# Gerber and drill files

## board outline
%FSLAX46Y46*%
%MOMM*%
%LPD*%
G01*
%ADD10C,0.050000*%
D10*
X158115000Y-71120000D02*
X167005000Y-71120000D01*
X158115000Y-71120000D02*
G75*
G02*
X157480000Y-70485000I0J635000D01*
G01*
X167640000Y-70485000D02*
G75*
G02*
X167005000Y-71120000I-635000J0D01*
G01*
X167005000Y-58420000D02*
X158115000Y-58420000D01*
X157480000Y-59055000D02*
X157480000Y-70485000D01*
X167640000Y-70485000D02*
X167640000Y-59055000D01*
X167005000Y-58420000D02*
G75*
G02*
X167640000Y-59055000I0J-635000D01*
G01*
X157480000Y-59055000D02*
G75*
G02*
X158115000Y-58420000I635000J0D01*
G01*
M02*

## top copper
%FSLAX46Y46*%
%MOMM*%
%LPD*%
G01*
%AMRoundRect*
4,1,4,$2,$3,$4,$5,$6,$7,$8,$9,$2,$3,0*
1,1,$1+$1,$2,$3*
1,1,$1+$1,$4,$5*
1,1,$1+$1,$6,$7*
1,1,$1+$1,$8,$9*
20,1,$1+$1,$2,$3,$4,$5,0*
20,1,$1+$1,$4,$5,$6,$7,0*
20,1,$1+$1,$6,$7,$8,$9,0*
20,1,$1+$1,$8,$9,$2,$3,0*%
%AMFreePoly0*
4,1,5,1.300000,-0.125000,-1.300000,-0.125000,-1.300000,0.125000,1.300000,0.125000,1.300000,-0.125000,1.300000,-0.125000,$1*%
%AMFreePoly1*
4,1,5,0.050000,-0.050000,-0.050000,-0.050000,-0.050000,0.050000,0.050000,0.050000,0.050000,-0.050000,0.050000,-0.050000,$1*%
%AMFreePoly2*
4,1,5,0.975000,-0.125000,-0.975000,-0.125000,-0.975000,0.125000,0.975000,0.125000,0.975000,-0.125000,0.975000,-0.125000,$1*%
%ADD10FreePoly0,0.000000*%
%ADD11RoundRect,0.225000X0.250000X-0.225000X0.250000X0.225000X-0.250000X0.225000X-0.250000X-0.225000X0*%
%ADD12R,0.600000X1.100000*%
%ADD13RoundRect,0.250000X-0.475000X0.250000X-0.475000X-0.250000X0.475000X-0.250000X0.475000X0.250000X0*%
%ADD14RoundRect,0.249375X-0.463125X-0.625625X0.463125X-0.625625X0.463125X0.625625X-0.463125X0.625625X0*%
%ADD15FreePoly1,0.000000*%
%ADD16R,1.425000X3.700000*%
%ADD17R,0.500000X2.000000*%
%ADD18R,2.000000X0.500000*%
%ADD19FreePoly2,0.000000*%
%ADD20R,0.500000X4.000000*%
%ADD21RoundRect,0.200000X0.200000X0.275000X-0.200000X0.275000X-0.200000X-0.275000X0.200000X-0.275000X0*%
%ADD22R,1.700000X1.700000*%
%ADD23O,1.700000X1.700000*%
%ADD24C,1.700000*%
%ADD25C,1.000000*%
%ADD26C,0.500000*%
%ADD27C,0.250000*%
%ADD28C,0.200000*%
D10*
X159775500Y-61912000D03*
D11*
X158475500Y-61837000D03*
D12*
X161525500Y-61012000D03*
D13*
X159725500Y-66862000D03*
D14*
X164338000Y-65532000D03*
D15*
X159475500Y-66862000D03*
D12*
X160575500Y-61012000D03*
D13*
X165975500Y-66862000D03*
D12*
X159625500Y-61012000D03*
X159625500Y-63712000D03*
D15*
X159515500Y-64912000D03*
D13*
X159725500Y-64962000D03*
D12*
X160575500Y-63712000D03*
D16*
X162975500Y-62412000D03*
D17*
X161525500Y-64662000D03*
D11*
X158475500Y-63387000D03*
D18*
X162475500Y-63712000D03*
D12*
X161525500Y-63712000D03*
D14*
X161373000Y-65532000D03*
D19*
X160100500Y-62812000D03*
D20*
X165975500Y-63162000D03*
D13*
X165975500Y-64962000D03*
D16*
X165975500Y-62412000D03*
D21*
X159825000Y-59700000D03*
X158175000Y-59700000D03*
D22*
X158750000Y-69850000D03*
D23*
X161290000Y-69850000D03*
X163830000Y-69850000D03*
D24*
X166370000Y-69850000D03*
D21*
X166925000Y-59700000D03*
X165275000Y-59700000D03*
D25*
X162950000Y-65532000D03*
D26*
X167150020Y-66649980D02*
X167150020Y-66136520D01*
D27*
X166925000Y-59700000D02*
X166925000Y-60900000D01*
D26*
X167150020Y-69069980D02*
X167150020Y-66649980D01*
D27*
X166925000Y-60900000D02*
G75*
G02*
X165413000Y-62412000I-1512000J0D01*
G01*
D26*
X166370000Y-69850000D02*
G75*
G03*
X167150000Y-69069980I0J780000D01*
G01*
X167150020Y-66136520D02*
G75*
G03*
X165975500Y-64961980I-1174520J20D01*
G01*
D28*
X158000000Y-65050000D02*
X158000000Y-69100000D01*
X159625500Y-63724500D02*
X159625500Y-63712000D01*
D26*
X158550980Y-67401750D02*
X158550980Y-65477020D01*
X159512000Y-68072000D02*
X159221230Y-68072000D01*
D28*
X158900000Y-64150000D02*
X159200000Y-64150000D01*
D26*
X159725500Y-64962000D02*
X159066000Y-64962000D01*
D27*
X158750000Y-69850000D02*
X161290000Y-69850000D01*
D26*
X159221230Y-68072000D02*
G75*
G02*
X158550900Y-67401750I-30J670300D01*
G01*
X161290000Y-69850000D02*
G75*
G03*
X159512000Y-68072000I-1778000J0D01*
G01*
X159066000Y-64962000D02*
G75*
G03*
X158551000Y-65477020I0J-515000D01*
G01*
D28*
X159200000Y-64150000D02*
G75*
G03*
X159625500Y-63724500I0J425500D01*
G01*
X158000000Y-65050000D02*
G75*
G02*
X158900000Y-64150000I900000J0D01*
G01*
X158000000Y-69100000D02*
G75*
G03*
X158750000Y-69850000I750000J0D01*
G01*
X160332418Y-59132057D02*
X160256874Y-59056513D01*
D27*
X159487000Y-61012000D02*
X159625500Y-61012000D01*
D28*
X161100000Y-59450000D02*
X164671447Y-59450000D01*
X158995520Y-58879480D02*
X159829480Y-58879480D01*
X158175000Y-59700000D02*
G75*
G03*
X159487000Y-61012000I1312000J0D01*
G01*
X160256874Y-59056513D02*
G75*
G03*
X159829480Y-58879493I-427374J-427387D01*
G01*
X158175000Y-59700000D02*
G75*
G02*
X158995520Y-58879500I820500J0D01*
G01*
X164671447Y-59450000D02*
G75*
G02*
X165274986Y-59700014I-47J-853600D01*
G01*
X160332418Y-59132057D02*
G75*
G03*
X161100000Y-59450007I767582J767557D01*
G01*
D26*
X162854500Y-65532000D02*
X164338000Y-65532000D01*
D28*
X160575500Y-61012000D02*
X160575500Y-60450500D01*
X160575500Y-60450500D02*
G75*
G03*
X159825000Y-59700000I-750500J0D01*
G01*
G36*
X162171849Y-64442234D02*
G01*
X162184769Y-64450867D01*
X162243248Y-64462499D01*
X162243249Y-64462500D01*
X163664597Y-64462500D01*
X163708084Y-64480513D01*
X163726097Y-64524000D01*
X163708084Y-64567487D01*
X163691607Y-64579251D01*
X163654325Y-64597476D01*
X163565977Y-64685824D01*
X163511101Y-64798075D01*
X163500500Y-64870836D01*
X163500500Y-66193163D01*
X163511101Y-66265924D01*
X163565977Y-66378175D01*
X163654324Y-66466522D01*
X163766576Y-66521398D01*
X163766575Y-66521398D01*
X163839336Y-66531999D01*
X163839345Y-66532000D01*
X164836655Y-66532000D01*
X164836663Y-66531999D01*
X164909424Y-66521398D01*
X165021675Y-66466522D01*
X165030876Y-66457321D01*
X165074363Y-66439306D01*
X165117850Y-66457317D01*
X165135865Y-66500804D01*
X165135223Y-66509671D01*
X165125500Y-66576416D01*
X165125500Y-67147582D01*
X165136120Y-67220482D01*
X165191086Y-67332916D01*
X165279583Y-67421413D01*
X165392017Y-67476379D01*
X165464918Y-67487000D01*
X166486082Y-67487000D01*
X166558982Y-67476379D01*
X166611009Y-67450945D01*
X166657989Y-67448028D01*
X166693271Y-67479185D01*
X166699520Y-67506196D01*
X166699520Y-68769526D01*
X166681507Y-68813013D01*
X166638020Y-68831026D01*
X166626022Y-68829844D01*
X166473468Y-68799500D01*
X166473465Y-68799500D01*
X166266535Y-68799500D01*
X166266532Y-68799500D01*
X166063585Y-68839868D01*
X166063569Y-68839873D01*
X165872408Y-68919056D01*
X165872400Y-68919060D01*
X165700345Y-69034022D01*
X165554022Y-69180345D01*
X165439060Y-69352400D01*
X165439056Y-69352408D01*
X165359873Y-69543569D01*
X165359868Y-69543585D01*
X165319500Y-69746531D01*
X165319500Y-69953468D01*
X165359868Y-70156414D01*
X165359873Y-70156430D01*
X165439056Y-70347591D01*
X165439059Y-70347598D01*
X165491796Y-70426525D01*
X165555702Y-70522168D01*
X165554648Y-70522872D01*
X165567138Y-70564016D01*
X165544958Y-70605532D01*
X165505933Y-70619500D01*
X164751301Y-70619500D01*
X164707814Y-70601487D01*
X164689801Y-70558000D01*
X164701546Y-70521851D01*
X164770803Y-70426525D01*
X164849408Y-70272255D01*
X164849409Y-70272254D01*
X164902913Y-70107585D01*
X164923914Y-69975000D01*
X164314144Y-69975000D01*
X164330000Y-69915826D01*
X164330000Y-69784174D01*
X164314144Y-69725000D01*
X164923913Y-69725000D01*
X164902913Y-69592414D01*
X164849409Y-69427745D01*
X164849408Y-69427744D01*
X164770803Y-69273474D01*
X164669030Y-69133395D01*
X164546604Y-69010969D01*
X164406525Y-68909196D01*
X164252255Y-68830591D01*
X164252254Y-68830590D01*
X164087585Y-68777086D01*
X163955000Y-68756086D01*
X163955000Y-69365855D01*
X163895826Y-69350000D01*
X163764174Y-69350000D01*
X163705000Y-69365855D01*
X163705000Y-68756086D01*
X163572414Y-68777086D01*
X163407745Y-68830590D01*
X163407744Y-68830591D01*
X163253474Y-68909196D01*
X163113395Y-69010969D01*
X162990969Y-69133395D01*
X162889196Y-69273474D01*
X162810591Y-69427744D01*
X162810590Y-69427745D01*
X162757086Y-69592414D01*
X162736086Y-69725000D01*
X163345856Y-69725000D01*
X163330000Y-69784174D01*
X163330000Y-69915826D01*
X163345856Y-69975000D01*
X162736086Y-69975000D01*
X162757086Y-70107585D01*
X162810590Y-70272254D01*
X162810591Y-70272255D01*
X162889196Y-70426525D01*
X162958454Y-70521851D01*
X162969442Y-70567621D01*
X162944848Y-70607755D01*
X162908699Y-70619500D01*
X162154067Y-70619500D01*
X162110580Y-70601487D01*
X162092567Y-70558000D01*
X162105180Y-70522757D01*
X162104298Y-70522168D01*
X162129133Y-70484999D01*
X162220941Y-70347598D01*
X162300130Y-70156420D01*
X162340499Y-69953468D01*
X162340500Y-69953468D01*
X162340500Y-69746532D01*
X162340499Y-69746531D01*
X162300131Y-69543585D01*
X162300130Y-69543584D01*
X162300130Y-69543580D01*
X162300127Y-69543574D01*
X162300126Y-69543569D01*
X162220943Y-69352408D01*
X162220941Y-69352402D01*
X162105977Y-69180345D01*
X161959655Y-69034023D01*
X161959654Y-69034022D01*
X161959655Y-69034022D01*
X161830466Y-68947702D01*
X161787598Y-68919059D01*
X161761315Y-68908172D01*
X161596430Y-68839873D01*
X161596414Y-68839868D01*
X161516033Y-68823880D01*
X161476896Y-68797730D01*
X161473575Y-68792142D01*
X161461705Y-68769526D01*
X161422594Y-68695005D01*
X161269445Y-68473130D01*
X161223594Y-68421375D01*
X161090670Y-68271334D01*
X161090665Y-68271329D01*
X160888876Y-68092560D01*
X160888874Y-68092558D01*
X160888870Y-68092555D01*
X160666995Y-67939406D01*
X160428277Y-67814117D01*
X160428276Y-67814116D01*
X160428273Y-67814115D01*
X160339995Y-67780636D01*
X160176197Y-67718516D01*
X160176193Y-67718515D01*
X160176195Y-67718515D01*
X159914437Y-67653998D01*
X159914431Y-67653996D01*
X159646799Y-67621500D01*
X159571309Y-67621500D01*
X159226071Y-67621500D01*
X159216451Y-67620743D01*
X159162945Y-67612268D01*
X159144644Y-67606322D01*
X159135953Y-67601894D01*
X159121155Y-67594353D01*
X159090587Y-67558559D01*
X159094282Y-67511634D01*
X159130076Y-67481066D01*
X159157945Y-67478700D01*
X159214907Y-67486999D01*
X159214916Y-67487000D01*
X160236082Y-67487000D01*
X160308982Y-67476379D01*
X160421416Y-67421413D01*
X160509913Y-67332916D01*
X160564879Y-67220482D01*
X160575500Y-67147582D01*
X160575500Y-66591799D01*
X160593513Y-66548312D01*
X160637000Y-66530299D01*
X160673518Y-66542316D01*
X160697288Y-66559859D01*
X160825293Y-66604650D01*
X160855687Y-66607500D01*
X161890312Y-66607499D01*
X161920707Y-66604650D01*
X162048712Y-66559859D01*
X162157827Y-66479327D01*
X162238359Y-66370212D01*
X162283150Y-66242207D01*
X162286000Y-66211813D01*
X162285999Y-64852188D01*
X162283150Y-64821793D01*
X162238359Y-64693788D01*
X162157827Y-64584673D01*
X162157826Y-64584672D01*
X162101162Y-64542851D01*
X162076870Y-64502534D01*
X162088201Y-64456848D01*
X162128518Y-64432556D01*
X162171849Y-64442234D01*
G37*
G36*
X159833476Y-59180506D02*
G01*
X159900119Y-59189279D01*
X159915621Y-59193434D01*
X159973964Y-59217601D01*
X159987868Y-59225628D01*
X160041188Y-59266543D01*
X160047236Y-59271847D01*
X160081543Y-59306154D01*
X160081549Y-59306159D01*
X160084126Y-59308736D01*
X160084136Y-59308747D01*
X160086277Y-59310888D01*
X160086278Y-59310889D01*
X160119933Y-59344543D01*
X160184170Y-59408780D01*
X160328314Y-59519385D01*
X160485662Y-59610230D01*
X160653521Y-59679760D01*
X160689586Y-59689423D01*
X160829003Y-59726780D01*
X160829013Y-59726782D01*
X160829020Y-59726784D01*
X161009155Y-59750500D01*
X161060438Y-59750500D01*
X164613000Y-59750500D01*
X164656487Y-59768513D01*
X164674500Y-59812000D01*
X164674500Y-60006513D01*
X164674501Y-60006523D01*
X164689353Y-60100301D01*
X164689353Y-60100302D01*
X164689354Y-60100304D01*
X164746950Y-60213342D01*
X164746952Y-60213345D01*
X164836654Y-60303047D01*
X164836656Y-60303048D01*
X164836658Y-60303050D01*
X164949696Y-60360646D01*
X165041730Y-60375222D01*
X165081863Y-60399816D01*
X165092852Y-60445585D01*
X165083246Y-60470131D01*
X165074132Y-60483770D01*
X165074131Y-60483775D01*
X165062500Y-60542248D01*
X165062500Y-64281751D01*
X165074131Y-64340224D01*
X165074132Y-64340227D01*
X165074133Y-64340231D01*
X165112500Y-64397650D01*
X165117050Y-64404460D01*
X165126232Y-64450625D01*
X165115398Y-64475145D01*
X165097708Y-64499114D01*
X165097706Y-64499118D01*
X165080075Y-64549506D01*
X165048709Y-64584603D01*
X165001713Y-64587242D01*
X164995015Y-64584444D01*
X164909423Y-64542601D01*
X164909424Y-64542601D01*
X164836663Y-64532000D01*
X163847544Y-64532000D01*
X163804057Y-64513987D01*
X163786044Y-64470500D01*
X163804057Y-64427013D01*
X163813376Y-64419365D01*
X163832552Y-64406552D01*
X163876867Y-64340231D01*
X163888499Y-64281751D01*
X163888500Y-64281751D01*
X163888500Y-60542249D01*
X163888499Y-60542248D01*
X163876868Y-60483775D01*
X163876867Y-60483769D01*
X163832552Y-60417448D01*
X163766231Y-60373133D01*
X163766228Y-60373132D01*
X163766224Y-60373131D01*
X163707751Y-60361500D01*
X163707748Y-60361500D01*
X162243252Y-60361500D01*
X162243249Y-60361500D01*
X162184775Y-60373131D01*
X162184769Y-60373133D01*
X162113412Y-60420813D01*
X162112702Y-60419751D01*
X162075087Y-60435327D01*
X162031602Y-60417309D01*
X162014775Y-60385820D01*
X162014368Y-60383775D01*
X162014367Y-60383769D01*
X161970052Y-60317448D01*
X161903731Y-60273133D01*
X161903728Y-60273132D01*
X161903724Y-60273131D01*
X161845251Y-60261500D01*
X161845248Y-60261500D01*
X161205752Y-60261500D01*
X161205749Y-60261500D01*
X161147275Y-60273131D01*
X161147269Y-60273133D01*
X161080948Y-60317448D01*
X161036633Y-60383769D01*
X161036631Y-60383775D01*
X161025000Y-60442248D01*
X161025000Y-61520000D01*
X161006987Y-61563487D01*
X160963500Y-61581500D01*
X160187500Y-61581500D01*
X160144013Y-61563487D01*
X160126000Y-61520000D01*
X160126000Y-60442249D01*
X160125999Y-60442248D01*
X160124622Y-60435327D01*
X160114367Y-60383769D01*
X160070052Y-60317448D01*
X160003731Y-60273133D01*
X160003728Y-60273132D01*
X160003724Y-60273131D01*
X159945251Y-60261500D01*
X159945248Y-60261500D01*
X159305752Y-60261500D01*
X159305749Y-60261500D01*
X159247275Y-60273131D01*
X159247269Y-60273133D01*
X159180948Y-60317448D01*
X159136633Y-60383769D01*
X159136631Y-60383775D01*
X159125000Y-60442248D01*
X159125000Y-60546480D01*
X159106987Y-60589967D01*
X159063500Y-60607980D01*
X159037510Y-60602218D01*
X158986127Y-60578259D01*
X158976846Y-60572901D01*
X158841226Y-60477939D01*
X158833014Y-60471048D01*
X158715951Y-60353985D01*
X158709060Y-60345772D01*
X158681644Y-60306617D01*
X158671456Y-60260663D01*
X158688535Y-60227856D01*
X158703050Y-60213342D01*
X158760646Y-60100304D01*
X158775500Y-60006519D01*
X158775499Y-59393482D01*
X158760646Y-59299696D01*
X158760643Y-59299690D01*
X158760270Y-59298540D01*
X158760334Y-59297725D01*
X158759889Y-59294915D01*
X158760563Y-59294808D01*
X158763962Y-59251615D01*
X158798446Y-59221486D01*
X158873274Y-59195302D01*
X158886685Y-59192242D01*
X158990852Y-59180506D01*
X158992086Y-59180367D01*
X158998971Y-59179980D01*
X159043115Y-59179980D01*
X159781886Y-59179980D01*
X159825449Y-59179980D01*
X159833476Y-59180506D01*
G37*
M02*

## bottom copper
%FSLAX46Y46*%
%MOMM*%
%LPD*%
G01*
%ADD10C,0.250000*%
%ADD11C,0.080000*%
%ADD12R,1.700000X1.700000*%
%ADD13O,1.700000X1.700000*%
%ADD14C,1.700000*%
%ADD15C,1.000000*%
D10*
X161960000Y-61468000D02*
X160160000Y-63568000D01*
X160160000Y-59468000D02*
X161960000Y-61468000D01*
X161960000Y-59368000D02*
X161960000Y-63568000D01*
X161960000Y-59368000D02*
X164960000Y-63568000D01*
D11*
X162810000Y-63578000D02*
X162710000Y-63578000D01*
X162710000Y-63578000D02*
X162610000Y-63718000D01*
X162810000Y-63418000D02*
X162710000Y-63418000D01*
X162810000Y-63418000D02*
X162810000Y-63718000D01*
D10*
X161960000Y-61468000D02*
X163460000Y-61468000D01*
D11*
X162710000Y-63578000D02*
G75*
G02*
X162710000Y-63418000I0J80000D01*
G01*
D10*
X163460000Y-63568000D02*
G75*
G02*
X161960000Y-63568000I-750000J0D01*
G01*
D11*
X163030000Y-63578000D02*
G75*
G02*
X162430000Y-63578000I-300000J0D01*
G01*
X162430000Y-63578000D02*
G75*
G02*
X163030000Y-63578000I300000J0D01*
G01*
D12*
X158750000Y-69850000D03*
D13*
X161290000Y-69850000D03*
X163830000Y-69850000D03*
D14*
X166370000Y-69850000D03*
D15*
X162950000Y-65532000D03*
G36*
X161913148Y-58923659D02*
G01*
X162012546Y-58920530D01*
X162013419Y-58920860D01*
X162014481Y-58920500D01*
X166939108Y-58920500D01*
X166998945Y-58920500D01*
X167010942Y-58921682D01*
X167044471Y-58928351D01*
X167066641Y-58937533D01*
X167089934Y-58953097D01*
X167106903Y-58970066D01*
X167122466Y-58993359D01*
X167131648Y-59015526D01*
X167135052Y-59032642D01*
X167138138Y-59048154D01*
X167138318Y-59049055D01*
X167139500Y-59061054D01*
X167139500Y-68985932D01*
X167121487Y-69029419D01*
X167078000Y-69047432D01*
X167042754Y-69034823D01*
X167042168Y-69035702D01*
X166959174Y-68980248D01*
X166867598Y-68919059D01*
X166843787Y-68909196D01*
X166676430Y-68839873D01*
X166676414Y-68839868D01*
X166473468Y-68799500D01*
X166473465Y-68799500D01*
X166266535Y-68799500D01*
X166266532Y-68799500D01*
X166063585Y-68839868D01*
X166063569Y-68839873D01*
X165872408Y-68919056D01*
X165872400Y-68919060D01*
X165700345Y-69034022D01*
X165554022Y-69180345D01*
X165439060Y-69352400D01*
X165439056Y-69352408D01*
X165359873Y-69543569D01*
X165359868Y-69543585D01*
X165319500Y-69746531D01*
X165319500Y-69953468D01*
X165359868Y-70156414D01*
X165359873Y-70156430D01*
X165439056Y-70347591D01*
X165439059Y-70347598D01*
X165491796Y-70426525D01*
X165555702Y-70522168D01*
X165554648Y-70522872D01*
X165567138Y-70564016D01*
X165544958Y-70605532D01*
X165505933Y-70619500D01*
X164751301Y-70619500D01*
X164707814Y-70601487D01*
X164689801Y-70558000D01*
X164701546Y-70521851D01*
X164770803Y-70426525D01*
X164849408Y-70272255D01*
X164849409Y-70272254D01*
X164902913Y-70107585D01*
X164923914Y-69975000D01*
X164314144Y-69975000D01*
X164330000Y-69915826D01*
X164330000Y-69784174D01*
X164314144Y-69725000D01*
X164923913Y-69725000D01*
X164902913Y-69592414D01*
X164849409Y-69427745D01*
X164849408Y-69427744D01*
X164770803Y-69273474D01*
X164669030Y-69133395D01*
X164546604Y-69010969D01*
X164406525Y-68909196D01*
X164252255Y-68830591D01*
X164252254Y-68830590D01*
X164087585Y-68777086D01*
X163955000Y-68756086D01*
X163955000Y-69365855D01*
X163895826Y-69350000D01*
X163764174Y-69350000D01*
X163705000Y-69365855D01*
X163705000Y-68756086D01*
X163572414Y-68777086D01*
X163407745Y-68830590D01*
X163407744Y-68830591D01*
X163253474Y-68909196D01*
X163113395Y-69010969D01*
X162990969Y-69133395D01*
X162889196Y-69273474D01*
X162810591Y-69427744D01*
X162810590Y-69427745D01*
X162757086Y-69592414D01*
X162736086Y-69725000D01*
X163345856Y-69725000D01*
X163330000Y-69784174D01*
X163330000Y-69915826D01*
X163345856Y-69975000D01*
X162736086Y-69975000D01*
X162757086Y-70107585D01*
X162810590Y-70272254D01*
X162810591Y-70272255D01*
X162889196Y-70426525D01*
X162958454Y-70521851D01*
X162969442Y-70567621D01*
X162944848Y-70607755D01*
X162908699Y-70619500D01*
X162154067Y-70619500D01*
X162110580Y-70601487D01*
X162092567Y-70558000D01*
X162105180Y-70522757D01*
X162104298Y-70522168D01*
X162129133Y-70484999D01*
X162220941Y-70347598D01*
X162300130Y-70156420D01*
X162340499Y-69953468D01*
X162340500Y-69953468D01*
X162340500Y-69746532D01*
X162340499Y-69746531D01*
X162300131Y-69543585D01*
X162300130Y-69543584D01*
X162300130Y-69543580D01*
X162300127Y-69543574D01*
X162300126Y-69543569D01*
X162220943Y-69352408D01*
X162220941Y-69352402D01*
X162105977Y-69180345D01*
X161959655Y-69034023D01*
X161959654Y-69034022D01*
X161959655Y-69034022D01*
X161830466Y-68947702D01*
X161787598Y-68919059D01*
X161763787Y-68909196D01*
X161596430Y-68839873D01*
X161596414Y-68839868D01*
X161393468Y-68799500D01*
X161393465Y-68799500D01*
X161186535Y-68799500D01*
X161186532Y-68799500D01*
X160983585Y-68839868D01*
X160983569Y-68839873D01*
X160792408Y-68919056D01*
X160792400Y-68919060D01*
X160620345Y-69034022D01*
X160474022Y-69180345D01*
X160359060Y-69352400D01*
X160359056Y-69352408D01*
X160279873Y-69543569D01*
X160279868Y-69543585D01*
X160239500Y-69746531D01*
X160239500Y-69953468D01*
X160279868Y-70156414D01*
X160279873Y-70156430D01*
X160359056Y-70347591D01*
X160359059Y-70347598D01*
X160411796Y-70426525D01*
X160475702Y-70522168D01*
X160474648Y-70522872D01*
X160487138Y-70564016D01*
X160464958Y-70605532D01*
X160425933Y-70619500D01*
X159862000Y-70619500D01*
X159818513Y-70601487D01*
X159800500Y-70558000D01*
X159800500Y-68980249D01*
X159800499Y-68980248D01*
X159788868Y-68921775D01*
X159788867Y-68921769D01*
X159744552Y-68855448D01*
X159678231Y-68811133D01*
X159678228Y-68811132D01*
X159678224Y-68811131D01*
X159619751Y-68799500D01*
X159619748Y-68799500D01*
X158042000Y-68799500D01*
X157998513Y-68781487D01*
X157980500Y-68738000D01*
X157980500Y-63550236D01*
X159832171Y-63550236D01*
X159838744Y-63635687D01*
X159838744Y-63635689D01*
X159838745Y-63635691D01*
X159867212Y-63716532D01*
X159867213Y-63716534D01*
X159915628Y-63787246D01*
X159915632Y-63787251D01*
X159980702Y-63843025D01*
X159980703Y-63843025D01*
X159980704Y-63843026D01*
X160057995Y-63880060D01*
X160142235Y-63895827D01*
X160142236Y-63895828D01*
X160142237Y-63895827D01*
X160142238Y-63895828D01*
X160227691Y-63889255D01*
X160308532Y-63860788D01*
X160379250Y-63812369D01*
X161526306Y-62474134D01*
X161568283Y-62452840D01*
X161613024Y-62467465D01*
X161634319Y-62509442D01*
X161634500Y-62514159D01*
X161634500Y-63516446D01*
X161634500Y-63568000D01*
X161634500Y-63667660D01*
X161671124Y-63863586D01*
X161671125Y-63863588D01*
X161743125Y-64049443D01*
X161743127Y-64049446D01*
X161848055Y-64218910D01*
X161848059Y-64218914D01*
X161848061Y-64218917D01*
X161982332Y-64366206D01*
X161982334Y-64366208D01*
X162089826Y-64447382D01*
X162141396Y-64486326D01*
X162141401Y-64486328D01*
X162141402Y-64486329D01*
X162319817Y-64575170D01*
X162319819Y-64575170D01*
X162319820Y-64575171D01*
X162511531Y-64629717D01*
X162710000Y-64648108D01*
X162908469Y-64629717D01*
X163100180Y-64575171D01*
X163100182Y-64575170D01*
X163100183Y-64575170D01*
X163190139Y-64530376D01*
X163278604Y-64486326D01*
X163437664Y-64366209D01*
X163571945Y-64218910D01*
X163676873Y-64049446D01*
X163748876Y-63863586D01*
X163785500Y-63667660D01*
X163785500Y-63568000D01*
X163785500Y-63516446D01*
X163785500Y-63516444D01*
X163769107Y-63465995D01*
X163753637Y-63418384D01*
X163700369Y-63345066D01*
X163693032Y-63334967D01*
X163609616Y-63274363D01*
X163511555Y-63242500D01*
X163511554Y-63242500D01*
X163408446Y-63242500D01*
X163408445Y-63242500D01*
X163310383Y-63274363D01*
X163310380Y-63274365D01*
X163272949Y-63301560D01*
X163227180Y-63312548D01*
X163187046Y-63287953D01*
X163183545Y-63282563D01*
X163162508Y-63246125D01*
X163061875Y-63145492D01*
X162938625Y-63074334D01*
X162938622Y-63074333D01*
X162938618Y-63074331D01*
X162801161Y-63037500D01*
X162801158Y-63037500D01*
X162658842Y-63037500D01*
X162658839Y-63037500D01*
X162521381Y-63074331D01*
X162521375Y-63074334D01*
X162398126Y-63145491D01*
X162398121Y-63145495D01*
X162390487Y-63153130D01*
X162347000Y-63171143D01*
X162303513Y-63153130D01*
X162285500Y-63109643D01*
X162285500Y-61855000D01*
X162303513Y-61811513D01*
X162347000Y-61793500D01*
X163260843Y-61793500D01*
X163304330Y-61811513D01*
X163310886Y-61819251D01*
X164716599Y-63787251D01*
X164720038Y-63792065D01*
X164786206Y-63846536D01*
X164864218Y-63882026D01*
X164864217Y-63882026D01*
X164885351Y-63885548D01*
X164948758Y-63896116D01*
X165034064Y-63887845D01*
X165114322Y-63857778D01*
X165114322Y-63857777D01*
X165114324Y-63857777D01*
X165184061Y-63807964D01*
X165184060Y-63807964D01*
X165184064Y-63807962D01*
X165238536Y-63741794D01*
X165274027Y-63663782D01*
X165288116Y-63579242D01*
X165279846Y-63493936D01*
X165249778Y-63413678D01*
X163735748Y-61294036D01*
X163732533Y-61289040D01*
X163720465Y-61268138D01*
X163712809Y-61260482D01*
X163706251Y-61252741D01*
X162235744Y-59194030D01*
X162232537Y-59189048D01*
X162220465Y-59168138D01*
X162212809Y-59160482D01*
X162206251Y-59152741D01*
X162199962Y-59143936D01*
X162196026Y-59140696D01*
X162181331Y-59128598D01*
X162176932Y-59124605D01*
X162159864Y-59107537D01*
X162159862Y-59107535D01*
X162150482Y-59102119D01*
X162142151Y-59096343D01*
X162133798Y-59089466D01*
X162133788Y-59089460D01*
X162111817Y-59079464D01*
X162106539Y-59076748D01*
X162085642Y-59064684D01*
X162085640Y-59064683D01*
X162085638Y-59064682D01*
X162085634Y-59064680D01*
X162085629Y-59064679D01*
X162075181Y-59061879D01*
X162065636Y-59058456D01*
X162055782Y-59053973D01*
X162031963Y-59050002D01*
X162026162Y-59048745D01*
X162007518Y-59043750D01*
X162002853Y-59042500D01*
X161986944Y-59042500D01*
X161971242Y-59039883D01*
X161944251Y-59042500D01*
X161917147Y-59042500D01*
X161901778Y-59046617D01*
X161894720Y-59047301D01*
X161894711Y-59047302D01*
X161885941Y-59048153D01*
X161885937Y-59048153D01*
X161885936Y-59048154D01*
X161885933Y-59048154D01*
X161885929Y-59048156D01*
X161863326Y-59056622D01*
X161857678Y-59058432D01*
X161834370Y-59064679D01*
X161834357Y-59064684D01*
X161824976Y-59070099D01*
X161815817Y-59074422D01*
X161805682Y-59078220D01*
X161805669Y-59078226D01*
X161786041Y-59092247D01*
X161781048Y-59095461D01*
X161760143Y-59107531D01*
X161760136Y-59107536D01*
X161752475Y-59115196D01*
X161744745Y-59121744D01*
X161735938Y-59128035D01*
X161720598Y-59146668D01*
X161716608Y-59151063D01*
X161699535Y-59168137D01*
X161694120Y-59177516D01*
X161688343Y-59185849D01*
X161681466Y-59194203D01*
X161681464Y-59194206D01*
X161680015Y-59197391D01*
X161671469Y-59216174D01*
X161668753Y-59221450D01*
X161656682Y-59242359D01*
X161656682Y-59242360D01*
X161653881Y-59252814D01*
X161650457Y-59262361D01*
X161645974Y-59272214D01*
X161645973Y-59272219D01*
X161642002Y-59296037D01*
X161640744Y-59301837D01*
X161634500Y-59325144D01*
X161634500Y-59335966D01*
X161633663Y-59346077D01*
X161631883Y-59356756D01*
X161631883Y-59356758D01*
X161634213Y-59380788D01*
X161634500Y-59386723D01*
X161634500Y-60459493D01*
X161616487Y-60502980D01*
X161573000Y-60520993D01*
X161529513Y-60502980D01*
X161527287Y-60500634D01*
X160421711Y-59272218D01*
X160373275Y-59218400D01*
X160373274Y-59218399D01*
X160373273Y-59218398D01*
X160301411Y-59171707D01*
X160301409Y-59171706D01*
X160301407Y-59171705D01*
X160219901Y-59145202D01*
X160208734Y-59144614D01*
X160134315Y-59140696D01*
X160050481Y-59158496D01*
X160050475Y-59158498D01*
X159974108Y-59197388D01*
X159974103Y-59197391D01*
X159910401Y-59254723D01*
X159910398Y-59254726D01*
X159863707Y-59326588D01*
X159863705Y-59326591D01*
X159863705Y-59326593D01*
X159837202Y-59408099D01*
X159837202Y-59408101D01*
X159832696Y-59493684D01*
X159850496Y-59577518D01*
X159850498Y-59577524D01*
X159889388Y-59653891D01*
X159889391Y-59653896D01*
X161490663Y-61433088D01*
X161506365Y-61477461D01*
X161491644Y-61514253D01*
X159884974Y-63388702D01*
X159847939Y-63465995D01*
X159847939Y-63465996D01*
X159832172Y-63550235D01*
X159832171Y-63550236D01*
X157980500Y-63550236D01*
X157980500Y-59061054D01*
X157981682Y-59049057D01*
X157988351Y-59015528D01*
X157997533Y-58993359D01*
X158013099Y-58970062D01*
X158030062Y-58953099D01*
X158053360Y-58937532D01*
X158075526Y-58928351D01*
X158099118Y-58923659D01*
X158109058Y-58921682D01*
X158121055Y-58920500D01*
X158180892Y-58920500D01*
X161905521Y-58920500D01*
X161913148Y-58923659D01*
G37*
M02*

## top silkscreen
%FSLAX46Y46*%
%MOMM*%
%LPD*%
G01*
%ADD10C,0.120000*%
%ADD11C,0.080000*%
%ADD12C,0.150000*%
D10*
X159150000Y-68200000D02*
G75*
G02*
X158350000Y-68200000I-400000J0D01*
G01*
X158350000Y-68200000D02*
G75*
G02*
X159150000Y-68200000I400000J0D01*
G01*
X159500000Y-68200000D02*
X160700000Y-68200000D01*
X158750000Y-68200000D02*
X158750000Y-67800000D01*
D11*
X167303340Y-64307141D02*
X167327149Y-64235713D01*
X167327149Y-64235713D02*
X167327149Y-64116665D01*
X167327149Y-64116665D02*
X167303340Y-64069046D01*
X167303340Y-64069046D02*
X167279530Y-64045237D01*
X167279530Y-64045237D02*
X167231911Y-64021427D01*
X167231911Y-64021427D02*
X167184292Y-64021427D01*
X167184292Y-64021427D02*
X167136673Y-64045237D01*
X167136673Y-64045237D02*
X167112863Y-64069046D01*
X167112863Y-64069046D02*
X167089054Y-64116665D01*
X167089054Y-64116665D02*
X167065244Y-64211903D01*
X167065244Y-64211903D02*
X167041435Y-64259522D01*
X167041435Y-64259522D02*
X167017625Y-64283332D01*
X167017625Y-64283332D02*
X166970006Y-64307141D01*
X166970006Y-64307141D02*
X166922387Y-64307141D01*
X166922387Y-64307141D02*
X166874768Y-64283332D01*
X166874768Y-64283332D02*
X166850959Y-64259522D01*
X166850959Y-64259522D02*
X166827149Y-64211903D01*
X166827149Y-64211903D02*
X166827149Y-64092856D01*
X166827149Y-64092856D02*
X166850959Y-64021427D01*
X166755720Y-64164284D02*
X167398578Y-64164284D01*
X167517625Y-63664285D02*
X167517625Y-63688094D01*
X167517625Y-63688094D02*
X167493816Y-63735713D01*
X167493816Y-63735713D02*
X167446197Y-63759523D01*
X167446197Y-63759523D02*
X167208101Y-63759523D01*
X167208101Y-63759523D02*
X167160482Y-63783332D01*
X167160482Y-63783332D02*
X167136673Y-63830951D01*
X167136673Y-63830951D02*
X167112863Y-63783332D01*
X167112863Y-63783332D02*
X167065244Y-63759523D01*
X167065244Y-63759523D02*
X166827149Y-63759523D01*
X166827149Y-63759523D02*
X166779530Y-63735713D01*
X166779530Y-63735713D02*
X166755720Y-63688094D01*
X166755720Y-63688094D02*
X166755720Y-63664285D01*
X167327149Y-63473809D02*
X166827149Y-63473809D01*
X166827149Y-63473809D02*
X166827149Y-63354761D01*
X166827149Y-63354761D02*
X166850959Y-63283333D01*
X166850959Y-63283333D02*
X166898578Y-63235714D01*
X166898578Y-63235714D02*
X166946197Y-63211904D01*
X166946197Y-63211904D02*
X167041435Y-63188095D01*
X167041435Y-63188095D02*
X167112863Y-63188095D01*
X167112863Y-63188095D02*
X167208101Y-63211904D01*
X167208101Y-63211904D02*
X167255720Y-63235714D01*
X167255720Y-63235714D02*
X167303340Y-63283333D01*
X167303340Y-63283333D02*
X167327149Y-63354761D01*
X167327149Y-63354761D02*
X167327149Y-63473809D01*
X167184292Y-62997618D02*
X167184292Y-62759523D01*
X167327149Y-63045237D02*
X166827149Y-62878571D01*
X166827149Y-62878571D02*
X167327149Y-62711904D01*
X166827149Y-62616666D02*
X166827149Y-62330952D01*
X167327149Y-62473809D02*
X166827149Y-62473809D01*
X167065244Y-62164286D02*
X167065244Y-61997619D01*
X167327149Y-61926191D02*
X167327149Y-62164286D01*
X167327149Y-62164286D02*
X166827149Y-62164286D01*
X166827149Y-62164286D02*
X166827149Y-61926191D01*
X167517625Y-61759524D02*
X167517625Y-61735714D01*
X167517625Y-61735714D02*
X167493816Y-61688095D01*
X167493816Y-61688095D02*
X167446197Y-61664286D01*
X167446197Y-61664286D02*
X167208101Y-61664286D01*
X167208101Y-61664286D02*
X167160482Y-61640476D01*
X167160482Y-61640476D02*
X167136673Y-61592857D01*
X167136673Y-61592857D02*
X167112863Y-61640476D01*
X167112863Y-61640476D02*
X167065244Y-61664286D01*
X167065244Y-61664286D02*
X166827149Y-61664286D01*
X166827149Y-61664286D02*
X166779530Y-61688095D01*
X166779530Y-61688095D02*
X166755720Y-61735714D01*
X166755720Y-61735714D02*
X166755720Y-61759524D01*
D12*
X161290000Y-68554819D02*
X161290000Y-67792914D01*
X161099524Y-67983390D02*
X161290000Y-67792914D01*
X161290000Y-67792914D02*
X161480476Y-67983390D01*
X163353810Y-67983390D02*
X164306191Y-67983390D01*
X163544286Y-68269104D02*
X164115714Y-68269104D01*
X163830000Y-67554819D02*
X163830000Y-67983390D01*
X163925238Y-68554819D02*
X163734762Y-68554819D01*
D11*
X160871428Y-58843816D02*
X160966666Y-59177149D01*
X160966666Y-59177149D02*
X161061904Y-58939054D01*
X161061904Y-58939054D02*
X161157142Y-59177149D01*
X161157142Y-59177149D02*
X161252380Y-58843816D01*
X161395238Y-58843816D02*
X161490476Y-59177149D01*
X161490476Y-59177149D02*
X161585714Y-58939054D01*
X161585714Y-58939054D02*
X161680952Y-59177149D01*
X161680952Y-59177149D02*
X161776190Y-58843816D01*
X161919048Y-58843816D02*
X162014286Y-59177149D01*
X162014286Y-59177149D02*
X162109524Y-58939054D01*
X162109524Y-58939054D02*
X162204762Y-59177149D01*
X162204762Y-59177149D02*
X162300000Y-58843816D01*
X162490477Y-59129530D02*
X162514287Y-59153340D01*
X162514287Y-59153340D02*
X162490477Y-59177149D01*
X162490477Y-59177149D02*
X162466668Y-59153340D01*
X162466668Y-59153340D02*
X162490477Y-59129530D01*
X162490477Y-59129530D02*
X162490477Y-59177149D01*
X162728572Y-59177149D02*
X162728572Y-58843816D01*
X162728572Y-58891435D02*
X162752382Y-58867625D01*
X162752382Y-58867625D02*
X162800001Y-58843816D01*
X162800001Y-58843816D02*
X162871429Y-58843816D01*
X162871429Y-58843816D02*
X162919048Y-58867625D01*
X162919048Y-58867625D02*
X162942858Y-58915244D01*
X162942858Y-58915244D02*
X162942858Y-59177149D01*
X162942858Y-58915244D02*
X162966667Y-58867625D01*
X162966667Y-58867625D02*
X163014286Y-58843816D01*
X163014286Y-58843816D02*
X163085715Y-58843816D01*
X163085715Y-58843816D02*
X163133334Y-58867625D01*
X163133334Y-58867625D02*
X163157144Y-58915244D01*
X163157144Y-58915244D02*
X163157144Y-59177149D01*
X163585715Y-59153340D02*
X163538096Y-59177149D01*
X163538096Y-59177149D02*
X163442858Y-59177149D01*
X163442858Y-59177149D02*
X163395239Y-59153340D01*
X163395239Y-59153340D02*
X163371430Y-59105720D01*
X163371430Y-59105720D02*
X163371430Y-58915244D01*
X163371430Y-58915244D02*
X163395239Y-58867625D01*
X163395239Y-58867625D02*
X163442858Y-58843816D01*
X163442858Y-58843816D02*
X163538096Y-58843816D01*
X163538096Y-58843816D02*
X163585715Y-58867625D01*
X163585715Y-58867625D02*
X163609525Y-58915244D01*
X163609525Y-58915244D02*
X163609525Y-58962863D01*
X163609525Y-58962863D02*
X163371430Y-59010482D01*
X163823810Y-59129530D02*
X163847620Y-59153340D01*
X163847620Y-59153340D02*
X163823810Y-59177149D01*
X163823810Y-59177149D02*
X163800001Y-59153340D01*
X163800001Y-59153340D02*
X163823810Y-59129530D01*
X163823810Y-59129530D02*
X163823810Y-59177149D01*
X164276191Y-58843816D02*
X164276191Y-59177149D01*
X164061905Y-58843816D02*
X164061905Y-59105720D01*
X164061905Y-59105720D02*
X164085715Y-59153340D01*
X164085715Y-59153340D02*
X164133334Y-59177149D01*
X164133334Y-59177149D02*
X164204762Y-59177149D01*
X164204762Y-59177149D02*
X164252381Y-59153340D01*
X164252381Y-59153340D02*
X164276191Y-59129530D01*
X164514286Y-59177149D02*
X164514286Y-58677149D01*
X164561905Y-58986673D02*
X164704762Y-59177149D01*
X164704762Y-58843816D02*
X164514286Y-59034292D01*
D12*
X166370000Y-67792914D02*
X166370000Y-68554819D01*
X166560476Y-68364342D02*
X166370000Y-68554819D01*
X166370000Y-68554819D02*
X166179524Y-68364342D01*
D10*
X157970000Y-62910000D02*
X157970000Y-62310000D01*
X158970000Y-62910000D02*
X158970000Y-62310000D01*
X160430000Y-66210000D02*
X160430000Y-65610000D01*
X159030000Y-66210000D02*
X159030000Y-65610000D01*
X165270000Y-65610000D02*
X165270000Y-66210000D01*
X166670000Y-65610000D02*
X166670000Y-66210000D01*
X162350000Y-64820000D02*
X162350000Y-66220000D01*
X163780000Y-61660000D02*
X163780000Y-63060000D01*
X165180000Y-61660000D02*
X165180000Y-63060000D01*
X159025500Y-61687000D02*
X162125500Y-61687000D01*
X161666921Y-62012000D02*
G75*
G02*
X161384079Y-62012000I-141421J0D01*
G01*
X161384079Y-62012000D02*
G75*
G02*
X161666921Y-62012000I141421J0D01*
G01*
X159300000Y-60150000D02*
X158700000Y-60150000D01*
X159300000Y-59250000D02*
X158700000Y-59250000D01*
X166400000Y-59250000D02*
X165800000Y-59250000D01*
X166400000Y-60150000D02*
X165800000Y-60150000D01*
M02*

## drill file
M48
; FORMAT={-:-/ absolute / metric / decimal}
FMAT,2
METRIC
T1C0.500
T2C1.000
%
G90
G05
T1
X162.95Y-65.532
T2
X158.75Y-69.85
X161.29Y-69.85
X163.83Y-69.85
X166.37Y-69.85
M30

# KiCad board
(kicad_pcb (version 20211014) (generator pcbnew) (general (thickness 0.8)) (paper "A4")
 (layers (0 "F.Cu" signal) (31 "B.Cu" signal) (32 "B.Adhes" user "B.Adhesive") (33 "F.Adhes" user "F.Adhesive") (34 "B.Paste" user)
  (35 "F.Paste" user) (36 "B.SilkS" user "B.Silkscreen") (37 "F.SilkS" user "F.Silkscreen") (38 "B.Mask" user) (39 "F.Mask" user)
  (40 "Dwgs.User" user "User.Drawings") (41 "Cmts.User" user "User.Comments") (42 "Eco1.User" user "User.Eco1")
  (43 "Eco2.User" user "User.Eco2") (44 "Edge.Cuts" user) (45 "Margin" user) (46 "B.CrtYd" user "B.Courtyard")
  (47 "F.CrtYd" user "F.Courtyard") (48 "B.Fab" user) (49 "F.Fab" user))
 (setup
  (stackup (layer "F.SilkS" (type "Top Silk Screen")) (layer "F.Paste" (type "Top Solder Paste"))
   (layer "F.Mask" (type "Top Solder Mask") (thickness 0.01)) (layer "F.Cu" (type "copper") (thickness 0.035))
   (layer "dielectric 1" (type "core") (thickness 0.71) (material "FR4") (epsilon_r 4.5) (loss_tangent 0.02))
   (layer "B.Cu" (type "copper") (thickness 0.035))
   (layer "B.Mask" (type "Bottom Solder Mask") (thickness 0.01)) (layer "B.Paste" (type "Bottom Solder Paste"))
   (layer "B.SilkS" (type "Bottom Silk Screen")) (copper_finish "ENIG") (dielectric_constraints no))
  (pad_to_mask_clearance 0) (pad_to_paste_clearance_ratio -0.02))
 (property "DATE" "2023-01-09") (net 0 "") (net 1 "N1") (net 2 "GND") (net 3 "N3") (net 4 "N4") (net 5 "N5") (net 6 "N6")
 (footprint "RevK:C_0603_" (layer "F.Cu") (at 158.47 62.61 90)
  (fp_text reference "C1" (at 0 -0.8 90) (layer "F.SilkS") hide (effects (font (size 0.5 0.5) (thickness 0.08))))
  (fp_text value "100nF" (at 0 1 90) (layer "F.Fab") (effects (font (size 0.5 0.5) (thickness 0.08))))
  (fp_line (start -0.3 -0.5) (end 0.3 -0.5) (layer "F.SilkS") (width 0.12))
  (fp_line (start -0.3 0.5) (end 0.3 0.5) (layer "F.SilkS") (width 0.12)))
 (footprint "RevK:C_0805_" (layer "F.Cu") (at 159.73 65.91 90)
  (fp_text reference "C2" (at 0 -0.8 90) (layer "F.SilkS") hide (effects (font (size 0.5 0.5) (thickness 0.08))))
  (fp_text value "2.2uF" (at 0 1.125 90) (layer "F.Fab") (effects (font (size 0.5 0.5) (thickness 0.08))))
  (fp_line (start -0.3 0.7) (end 0.3 0.7) (layer "F.SilkS") (width 0.12))
  (fp_line (start -0.3 -0.7) (end 0.3 -0.7) (layer "F.SilkS") (width 0.12)))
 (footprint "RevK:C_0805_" (layer "F.Cu") (at 165.97 65.91 -90)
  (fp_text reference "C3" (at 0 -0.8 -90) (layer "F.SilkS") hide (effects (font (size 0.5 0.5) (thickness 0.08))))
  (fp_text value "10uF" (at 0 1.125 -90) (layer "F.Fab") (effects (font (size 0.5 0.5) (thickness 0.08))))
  (fp_line (start -0.3 0.7) (end 0.3 0.7) (layer "F.SilkS") (width 0.12))
  (fp_line (start -0.3 -0.7) (end 0.3 -0.7) (layer "F.SilkS") (width 0.12)))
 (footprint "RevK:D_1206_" (layer "F.Cu") (at 162.85 65.52)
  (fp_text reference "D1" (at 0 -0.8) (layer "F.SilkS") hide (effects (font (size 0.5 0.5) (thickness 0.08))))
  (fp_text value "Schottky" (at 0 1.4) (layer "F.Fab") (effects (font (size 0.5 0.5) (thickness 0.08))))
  (fp_line (start -0.5 -0.7) (end -0.5 0.7) (layer "F.SilkS") (width 0.12)))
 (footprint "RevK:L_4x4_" (layer "F.Cu") (at 164.48 62.36)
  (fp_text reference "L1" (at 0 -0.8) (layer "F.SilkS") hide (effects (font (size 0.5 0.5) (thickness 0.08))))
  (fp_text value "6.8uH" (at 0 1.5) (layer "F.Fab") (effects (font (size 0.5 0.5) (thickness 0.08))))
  (fp_line (start -0.7 -0.7) (end -0.7 0.7) (layer "F.SilkS") (width 0.12))
  (fp_line (start 0.7 -0.7) (end 0.7 0.7) (layer "F.SilkS") (width 0.12)))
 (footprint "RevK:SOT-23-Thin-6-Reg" (layer "F.Cu") (at 160.5755 62.362)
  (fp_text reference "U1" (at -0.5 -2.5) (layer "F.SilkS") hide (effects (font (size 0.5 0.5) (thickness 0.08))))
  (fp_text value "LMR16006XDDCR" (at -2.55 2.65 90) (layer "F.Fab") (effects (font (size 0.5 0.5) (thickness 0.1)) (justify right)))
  (fp_line (start -1.55 -0.675) (end 1.55 -0.675) (layer "F.SilkS") (width 0.12))
  (fp_circle (center 0.95 -0.35) (end 1.05 -0.25) (layer "F.SilkS") (width 0.12) (fill none))
  (pad "" smd roundrect (at 5.4 0.05) (size 1.2 1) (layers "F.Paste") (roundrect_rratio 0.25))
  (pad "" smd roundrect (at 5.4 1.2) (size 1.2 1) (layers "F.Paste") (roundrect_rratio 0.25))
  (pad "" smd roundrect (at 2.4 0.05) (size 1.2 1) (layers "F.Paste") (roundrect_rratio 0.25))
  (pad "" smd roundrect (at 2.4 1.2) (size 1.2 1) (layers "F.Paste") (roundrect_rratio 0.25))
  (pad "" smd roundrect (at 2.4 -1.1) (size 1.2 1) (layers "F.Paste") (roundrect_rratio 0.25))
  (pad "" smd roundrect (at 5.4 -1.1) (size 1.2 1) (layers "F.Paste") (roundrect_rratio 0.25))
  (pad "1" smd custom (at -0.8 -0.45) (size 2.6 0.25) (layers "F.Cu") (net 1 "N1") (clearance 0.2)
   (options (clearance outline) (anchor rect)) (primitives))
  (pad "1" smd roundrect (at -2.1 -0.525 90) (size 0.9 0.95) (layers "F.Cu" "F.Paste" "F.Mask") (roundrect_rratio 0.25) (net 1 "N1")
   (clearance 0.2))
  (pad "1" smd rect (at 0.95 -1.35 90) (size 1.1 0.6) (layers "F.Cu" "F.Paste" "F.Mask") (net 1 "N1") (clearance 0.2))
  (pad "2" smd roundrect (at -0.85 4.5 270) (size 1 1.45) (layers "F.Cu" "F.Paste" "F.Mask") (roundrect_rratio 0.25) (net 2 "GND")
   (zone_connect 0))
  (pad "2" smd roundrect (at 3.7625 3.17) (size 1.425 1.75) (layers "F.Cu" "F.Paste" "F.Mask") (roundrect_rratio 0.175) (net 2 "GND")
   (clearance 0.2) (zone_connect 0))
  (pad "2" smd custom (at -1.1 4.5) (size 0.1 0.1) (layers "F.Cu") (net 2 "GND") (clearance 0.2) (zone_connect 0)
   (options (clearance outline) (anchor rect)) (primitives))
  (pad "2" smd rect (at 0 -1.35 90) (size 1.1 0.6) (layers "F.Cu" "F.Paste" "F.Mask") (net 2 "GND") (clearance 0.2))
  (pad "2" smd roundrect (at 5.4 4.5 270) (size 1 1.45) (layers "F.Cu" "F.Paste" "F.Mask") (roundrect_rratio 0.25) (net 2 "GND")
   (zone_connect 0))
  (pad "3" smd rect (at -0.95 -1.35 90) (size 1.1 0.6) (layers "F.Cu" "F.Paste" "F.Mask") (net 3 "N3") (clearance 0.2))
  (pad "4" smd rect (at -0.95 1.35 90) (size 1.1 0.6) (layers "F.Cu" "F.Paste" "F.Mask") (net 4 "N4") (clearance 0.2))
  (pad "5" smd custom (at -1.06 2.55) (size 0.1 0.1) (layers "F.Cu") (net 4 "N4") (zone_connect 0)
   (options (clearance outline) (anchor rect)) (primitives))
  (pad "5" smd roundrect (at -0.85 2.6 270) (size 1 1.45) (layers "F.Cu" "F.Paste" "F.Mask") (roundrect_rratio 0.25) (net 4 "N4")
   (clearance 0.2))
  (pad "5" smd rect (at 0 1.35 90) (size 1.1 0.6) (layers "F.Cu" "F.Paste" "F.Mask") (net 4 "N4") (clearance 0.2) (zone_connect 0))
  (pad "6" smd rect (at 2.4 0.05 90) (size 3.7 1.425) (layers "F.Cu" "F.Mask") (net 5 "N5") (clearance 0.2))
  (pad "6" smd rect (at 0.95 2.3 90) (size 2 0.5) (layers "F.Cu") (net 5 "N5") (clearance 0.2))
  (pad "6" smd roundrect (at -2.1 1.025 90) (size 0.9 0.95) (layers "F.Cu" "F.Paste" "F.Mask") (roundrect_rratio 0.25) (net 5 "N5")
   (clearance 0.2))
  (pad "6" smd rect (at 1.9 1.35) (size 2 0.5) (layers "F.Cu") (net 5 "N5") (clearance 0.2))
  (pad "6" smd rect (at 0.95 1.35 90) (size 1.1 0.6) (layers "F.Cu" "F.Paste" "F.Mask") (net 5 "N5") (clearance 0.2))
  (pad "6" smd roundrect (at 0.7975 3.17) (size 1.425 1.75) (layers "F.Cu" "F.Paste" "F.Mask") (roundrect_rratio 0.175) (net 5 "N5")
   (clearance 0.2))
  (pad "6" smd custom (at -0.475 0.45) (size 1.95 0.25) (layers "F.Cu") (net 5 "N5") (clearance 0.2)
   (options (clearance outline) (anchor rect)) (primitives))
  (pad "7" smd rect (at 5.4 0.8) (size 0.5 4) (layers "F.Cu") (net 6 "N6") (zone_connect 0))
  (pad "7" smd roundrect (at 5.4 2.6 270) (size 1 1.45) (layers "F.Cu" "F.Paste" "F.Mask") (roundrect_rratio 0.25) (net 6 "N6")
   (clearance 0.2) (zone_connect 0))
  (pad "7" smd rect (at 5.4 0.05 90) (size 3.7 1.425) (layers "F.Cu" "F.Mask") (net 6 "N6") (zone_connect 0)))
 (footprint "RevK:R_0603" (layer "F.Cu") (at 159 59.7 180)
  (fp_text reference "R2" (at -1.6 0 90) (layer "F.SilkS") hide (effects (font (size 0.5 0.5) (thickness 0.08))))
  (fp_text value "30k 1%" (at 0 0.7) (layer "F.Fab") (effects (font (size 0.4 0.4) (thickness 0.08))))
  (fp_line (start -0.3 -0.45) (end 0.3 -0.45) (layer "F.SilkS") (width 0.12))
  (fp_line (start -0.3 0.45) (end 0.3 0.45) (layer "F.SilkS") (width 0.12))
  (pad "1" smd roundrect (at -0.825 0 180) (size 0.8 0.95) (layers "F.Cu" "F.Paste" "F.Mask") (roundrect_rratio 0.25) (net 2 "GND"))
  (pad "2" smd roundrect (at 0.825 0 180) (size 0.8 0.95) (layers "F.Cu" "F.Paste" "F.Mask") (roundrect_rratio 0.25) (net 3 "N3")))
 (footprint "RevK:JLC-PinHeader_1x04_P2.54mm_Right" (layer "F.Cu") (at 162.56 69.85)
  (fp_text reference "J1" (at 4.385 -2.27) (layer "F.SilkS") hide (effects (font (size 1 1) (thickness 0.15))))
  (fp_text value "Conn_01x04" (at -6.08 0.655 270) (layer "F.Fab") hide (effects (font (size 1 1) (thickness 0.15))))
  (pad "1" thru_hole rect (at -3.81 0 270) (size 1.7 1.7) (drill 1) (layers *.Cu *.Mask) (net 4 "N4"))
  (pad "2" thru_hole oval (at -1.27 0 270) (size 1.7 1.7) (drill 1) (layers *.Cu *.Mask) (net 4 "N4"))
  (pad "3" thru_hole oval (at 1.27 0 270) (size 1.7 1.7) (drill 1) (layers *.Cu *.Mask) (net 2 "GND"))
  (pad "4" thru_hole circle (at 3.81 0 270) (size 1.7 1.7) (drill 1) (layers *.Cu *.Mask) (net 6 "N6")))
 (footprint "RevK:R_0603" (layer "F.Cu") (at 166.1 59.7 180)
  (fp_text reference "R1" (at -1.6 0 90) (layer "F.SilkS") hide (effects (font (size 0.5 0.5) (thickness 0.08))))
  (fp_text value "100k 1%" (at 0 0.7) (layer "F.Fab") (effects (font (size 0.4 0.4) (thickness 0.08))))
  (fp_line (start -0.3 0.45) (end 0.3 0.45) (layer "F.SilkS") (width 0.12))
  (fp_line (start -0.3 -0.45) (end 0.3 -0.45) (layer "F.SilkS") (width 0.12))
  (pad "1" smd roundrect (at -0.825 0 180) (size 0.8 0.95) (layers "F.Cu" "F.Paste" "F.Mask") (roundrect_rratio 0.25) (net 6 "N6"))
  (pad "2" smd roundrect (at 0.825 0 180) (size 0.8 0.95) (layers "F.Cu" "F.Paste" "F.Mask") (roundrect_rratio 0.25) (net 3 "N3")))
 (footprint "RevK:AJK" (layer "B.Cu") (at 161.96 61.468 180)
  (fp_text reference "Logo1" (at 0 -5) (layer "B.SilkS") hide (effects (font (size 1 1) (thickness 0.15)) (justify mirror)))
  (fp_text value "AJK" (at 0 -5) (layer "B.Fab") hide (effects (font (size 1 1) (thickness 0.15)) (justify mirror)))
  (fp_line (start 0 0) (end 1.8 -2.1) (layer "B.Cu") (width 0.25))
  (fp_line (start 1.8 2) (end 0 0) (layer "B.Cu") (width 0.25))
  (fp_line (start 0 2.1) (end 0 -2.1) (layer "B.Cu") (width 0.25))
  (fp_line (start 0 2.1) (end -3 -2.1) (layer "B.Cu") (width 0.25))
  (fp_line (start -0.85 -2.11) (end -0.75 -2.11) (layer "B.Cu") (width 0.08))
  (fp_line (start -0.75 -2.11) (end -0.65 -2.25) (layer "B.Cu") (width 0.08))
  (fp_line (start -0.85 -1.95) (end -0.75 -1.95) (layer "B.Cu") (width 0.08))
  (fp_line (start -0.85 -1.95) (end -0.85 -2.25) (layer "B.Cu") (width 0.08))
  (fp_line (start 0 0) (end -1.5 0) (layer "B.Cu") (width 0.25))
  (fp_arc (start -0.75 -2.11) (mid -0.67 -2.03) (end -0.75 -1.95) (layer "B.Cu") (width 0.08))
  (fp_arc (start -1.5 -2.1) (mid -0.75 -2.85) (end 0 -2.1) (layer "B.Cu") (width 0.25))
  (fp_circle (center -0.77 -2.11) (end -0.47 -2.11) (layer "B.Cu") (width 0.08) (fill none)))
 (gr_circle (center 158.75 68.2) (end 158.75 68.6) (layer "F.SilkS") (width 0.12) (fill none))
 (gr_line (start 159.5 68.2) (end 160.7 68.2) (layer "F.SilkS") (width 0.12))
 (gr_line (start 158.75 68.2) (end 158.75 67.8) (layer "F.SilkS") (width 0.12))
 (gr_line (start 158.115 71.12) (end 167.005 71.12) (layer "Edge.Cuts") (width 0.05))
 (gr_arc (start 158.115 71.12) (mid 157.665987 70.934013) (end 157.48 70.485) (layer "Edge.Cuts") (width 0.05))
 (gr_arc (start 167.64 70.485) (mid 167.454013 70.934013) (end 167.005 71.12) (layer "Edge.Cuts") (width 0.05))
 (gr_line (start 167.005 58.42) (end 158.115 58.42) (layer "Edge.Cuts") (width 0.05))
 (gr_line (start 157.48 59.055) (end 157.48 70.485) (layer "Edge.Cuts") (width 0.05))
 (gr_line (start 167.64 70.485) (end 167.64 59.055) (layer "Edge.Cuts") (width 0.05))
 (gr_arc (start 167.005 58.42) (mid 167.454013 58.605987) (end 167.64 59.055) (layer "Edge.Cuts") (width 0.05))
 (gr_arc (start 157.48 59.055) (mid 157.665987 58.605987) (end 158.115 58.42) (layer "Edge.Cuts") (width 0.05))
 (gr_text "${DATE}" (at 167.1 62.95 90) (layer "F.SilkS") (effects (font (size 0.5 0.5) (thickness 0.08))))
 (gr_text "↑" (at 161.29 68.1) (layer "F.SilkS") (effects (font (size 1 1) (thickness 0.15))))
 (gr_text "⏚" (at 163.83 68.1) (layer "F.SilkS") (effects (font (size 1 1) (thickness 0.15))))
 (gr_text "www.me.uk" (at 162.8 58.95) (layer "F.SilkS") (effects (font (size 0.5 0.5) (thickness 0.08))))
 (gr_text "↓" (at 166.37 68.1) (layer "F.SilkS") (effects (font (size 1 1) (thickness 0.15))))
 (segment (start 167.15002 66.64998) (end 167.15002 66.13652) (width 0.5) (layer "F.Cu") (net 6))
 (segment (start 166.925 59.7) (end 166.925 60.9) (width 0.25) (layer "F.Cu") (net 6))
 (segment (start 167.15002 69.06998) (end 167.15002 66.64998) (width 0.5) (layer "F.Cu") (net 6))
 (arc (start 166.925 60.9) (mid 166.482145 61.969145) (end 165.413 62.412) (width 0.25) (layer "F.Cu") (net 6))
 (arc (start 166.37 69.85) (mid 166.921557 69.621537) (end 167.15002 69.06998) (width 0.5) (layer "F.Cu") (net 6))
 (arc (start 167.15002 66.13652) (mid 166.806011 65.306009) (end 165.9755 64.962) (width 0.5) (layer "F.Cu") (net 6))
 (segment (start 158 65.05) (end 158 69.1) (width 0.2) (layer "F.Cu") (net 4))
 (segment (start 159.6255 63.7245) (end 159.6255 63.712) (width 0.2) (layer "F.Cu") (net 4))
 (segment (start 158.55098 67.40175) (end 158.55098 65.47702) (width 0.5) (layer "F.Cu") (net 4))
 (segment (start 159.512 68.072) (end 159.22123 68.072) (width 0.5) (layer "F.Cu") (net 4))
 (segment (start 158.9 64.15) (end 159.2 64.15) (width 0.2) (layer "F.Cu") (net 4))
 (segment (start 159.7255 64.962) (end 159.066 64.962) (width 0.5) (layer "F.Cu") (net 4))
 (segment (start 158.75 69.85) (end 161.29 69.85) (width 0.25) (layer "F.Cu") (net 4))
 (arc (start 159.22123 68.072) (mid 158.747292 67.875688) (end 158.55098 67.40175) (width 0.5) (layer "F.Cu") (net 4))
 (arc (start 161.29 69.85) (mid 160.769236 68.592764) (end 159.512 68.072) (width 0.5) (layer "F.Cu") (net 4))
 (arc (start 159.066 64.962) (mid 158.701826 65.112846) (end 158.55098 65.47702) (width 0.5) (layer "F.Cu") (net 4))
 (arc (start 159.2 64.15) (mid 159.500874 64.025374) (end 159.6255 63.7245) (width 0.2) (layer "F.Cu") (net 4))
 (arc (start 158 65.05) (mid 158.263604 64.413604) (end 158.9 64.15) (width 0.2) (layer "F.Cu") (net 4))
 (arc (start 158 69.1) (mid 158.21967 69.63033) (end 158.75 69.85) (width 0.2) (layer "F.Cu") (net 4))
 (segment (start 160.332418 59.132057) (end 160.256874 59.056513) (width 0.2) (layer "F.Cu") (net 3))
 (segment (start 159.487 61.012) (end 159.6255 61.012) (width 0.25) (layer "F.Cu") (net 3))
 (segment (start 161.1 59.45) (end 164.671447 59.45) (width 0.2) (layer "F.Cu") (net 3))
 (segment (start 158.99552 58.87948) (end 159.82948 58.87948) (width 0.2) (layer "F.Cu") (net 3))
 (arc (start 158.175 59.7) (mid 158.559276 60.627724) (end 159.487 61.012) (width 0.2) (layer "F.Cu") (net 3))
 (arc (start 160.256874 59.056513) (mid 160.060784 58.925489) (end 159.82948 58.87948) (width 0.2) (layer "F.Cu") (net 3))
 (arc (start 158.175 59.7) (mid 158.415325 59.119805) (end 158.99552 58.87948) (width 0.2) (layer "F.Cu") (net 3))
 (arc (start 164.671447 59.45) (mid 164.998087 59.514973) (end 165.275 59.7) (width 0.2) (layer "F.Cu") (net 3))
 (arc (start 160.332418 59.132057) (mid 160.684588 59.367369) (end 161.1 59.45) (width 0.2) (layer "F.Cu") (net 3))
 (segment (start 162.8545 65.532) (end 164.338 65.532) (width 0.5) (layer "F.Cu") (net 2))
 (segment (start 160.5755 61.012) (end 160.5755 60.4505) (width 0.2) (layer "F.Cu") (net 2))
 (via (at 162.95 65.532) (size 1) (drill 0.5) (layers "F.Cu" "B.Cu") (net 2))
 (arc (start 160.5755 60.4505) (mid 160.355684 59.919816) (end 159.825 59.7) (width 0.2) (layer "F.Cu") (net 2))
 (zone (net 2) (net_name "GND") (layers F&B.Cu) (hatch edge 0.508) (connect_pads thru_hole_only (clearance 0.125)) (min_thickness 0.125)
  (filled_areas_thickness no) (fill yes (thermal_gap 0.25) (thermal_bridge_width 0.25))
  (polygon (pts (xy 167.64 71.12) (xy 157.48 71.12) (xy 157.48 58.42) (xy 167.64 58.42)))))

